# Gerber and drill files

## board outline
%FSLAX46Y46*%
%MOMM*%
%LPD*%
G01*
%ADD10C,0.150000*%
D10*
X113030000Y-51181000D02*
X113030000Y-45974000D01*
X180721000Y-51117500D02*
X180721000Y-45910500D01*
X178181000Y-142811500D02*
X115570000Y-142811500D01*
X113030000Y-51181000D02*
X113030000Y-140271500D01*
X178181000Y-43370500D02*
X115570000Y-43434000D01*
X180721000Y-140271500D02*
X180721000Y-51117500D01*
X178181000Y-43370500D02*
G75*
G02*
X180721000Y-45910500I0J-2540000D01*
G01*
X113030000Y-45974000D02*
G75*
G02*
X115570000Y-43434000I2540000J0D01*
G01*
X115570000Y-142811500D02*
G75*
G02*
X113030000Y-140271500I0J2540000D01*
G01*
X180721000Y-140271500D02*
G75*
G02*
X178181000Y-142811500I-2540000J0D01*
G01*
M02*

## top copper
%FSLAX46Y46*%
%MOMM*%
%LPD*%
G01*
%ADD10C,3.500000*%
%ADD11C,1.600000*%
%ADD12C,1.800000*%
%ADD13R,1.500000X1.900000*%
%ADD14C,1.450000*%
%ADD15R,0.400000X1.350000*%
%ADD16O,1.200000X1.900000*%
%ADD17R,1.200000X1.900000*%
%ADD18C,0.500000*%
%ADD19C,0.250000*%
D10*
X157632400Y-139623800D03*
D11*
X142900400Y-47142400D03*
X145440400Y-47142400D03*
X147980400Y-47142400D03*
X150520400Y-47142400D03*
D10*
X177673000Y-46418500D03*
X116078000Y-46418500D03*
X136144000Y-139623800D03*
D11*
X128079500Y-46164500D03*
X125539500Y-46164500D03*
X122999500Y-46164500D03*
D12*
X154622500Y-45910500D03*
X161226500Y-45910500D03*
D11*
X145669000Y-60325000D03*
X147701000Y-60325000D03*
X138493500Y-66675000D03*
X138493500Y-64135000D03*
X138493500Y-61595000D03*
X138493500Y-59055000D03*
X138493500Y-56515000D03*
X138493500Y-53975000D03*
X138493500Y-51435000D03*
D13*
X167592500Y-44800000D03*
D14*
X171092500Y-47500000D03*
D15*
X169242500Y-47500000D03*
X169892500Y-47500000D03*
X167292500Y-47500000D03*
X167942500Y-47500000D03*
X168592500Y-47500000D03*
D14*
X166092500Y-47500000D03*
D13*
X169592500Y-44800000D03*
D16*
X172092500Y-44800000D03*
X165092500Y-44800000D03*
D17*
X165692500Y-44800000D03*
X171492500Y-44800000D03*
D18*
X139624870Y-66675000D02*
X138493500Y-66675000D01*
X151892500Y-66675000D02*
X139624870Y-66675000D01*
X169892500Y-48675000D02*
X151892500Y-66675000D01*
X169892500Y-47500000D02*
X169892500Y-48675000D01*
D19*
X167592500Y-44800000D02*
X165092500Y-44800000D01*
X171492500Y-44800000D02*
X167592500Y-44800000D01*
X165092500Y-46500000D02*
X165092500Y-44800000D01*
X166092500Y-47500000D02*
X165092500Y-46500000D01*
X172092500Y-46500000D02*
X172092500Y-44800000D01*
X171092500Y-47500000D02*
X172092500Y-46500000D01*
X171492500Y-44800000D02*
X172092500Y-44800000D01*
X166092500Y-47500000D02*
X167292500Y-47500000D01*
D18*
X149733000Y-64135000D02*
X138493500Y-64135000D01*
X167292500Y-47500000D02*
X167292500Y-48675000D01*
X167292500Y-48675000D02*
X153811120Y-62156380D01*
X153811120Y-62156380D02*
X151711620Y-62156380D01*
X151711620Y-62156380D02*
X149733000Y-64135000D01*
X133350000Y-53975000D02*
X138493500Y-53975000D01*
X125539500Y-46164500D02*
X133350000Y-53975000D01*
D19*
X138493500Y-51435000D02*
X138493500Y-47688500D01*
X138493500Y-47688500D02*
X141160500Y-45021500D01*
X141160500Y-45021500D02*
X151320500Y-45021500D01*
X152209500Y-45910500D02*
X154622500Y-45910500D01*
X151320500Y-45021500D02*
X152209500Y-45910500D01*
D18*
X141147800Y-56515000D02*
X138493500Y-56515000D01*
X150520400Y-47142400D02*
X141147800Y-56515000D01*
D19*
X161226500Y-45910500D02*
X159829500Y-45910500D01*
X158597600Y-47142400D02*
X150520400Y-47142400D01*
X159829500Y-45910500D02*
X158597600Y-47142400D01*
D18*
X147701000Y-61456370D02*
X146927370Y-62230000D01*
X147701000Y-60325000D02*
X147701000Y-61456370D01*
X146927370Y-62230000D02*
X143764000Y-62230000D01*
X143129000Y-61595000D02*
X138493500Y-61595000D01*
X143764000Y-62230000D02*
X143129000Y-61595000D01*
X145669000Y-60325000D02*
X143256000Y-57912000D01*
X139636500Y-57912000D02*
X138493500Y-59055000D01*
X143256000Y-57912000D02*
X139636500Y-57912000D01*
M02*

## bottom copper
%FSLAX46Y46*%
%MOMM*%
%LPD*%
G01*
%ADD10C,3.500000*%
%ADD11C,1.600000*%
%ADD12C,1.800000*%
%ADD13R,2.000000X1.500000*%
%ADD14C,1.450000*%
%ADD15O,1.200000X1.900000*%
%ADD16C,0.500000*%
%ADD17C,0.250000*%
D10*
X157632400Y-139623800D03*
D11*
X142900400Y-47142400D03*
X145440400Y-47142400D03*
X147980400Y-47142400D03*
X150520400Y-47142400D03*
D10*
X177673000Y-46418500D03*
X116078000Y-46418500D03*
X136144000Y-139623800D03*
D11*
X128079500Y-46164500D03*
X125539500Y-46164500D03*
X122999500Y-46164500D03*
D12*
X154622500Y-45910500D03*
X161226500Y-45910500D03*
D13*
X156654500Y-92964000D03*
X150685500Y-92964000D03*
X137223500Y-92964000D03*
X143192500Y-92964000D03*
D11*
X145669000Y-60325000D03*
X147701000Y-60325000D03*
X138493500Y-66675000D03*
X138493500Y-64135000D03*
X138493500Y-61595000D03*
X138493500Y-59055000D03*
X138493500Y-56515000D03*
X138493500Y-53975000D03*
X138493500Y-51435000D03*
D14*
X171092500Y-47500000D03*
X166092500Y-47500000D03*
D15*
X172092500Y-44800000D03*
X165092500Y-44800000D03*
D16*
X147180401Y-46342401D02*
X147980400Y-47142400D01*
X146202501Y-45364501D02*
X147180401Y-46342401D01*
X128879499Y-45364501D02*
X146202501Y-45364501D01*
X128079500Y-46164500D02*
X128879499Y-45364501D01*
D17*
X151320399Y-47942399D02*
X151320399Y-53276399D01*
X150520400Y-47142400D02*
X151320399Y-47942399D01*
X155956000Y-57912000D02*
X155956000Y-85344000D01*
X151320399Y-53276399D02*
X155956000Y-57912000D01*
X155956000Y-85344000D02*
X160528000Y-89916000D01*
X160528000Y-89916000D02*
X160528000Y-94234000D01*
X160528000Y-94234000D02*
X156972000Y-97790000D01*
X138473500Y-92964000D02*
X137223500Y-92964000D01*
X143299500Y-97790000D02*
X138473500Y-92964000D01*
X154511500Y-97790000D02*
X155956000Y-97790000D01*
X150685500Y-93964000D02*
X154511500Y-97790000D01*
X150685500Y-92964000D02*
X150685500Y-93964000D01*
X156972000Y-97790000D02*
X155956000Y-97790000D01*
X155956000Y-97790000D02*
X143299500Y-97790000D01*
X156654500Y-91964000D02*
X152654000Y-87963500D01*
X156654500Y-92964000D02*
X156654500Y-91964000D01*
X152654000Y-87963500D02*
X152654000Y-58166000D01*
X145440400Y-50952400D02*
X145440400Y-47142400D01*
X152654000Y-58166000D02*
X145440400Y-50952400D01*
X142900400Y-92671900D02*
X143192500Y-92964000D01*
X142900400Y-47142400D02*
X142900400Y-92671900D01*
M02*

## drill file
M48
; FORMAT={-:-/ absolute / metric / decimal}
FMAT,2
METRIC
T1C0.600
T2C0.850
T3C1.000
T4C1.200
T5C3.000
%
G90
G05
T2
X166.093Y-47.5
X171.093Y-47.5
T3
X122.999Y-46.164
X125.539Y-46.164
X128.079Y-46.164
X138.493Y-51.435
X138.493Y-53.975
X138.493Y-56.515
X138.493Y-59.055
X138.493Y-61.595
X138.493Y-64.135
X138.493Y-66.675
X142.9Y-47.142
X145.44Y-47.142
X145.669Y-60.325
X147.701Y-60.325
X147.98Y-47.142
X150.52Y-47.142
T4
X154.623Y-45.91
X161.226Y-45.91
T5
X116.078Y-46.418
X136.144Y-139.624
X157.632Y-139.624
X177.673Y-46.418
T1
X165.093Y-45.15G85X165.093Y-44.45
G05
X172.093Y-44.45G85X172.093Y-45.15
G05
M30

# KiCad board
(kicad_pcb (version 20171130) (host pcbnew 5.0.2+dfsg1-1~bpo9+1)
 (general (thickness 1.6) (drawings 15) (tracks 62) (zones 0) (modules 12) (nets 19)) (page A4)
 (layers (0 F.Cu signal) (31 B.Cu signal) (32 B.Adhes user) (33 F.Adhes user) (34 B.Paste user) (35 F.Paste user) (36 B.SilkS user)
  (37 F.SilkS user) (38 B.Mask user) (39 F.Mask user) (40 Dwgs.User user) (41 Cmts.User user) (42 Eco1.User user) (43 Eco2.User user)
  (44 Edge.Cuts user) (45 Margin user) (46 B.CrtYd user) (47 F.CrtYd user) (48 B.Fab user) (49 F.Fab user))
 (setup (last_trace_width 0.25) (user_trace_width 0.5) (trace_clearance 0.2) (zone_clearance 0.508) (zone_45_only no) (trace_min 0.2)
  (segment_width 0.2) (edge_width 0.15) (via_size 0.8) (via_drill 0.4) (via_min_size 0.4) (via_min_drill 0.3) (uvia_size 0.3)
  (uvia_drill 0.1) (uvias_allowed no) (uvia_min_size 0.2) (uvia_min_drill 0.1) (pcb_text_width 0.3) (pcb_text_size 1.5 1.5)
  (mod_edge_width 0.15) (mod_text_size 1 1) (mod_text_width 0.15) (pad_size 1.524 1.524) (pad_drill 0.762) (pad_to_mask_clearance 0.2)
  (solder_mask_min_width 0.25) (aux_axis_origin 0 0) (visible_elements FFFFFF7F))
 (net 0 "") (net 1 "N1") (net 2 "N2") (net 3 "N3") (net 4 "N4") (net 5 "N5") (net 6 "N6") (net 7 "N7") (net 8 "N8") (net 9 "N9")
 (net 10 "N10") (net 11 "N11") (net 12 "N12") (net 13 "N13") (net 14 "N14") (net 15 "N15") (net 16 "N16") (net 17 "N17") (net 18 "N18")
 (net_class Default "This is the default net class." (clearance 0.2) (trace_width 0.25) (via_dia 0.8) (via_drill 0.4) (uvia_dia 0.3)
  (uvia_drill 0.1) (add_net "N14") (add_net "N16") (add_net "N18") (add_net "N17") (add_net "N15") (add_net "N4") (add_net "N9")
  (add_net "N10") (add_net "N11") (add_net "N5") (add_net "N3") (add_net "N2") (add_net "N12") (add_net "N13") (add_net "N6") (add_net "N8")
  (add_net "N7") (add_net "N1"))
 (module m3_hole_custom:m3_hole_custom (layer F.Cu) (at 157.6324 139.6238)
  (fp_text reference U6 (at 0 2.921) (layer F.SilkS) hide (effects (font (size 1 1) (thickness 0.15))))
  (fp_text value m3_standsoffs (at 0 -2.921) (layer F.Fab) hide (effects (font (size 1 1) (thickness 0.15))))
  (pad 1 thru_hole circle (at 0 0) (size 3.5 3.5) (drill 3) (layers *.Cu *.Mask) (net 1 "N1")))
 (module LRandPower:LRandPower (layer F.Cu) (at 146.7104 47.1424)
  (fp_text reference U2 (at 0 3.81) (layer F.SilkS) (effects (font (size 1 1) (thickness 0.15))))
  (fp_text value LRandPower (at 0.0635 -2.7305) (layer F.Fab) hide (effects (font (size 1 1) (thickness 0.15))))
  (pad 1 thru_hole circle (at -3.81 0) (size 1.6 1.6) (drill 1) (layers *.Cu *.Mask) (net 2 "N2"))
  (pad 2 thru_hole circle (at -1.27 0) (size 1.6 1.6) (drill 1) (layers *.Cu *.Mask) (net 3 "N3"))
  (pad 3 thru_hole circle (at 1.27 0) (size 1.6 1.6) (drill 1) (layers *.Cu *.Mask) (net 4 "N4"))
  (pad 4 thru_hole circle (at 3.81 0) (size 1.6 1.6) (drill 1) (layers *.Cu *.Mask) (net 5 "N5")))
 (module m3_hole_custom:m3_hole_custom (layer F.Cu) (at 177.673 46.4185)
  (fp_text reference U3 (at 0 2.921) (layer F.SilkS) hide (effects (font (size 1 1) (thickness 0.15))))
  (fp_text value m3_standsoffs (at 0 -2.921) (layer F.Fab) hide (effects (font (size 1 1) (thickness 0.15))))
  (pad 1 thru_hole circle (at 0 0) (size 3.5 3.5) (drill 3) (layers *.Cu *.Mask) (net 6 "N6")))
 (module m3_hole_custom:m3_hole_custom (layer F.Cu) (at 116.078 46.4185)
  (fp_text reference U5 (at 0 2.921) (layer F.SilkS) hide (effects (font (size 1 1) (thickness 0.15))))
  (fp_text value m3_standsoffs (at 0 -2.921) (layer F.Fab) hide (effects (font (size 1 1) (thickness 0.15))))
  (pad 1 thru_hole circle (at 0 0) (size 3.5 3.5) (drill 3) (layers *.Cu *.Mask) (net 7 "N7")))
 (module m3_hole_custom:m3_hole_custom (layer F.Cu) (at 136.144 139.6238)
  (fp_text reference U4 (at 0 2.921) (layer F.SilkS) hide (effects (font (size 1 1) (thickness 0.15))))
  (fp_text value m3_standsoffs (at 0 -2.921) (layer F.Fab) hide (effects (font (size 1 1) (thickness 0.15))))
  (pad 1 thru_hole circle (at 0 0) (size 3.5 3.5) (drill 3) (layers *.Cu *.Mask) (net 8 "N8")))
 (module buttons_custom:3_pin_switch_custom (layer F.Cu) (at 125.5395 46.1645 180)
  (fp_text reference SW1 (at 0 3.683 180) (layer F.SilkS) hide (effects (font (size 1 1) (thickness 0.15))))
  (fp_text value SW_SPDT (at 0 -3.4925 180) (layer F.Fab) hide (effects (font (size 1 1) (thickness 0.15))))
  (pad 1 thru_hole circle (at -2.54 0 180) (size 1.6 1.6) (drill 1) (layers *.Cu *.Mask) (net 4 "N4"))
  (pad 2 thru_hole circle (at 0 0 180) (size 1.6 1.6) (drill 1) (layers *.Cu *.Mask) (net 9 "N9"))
  (pad 3 thru_hole circle (at 2.54 0 180) (size 1.6 1.6) (drill 1) (layers *.Cu *.Mask) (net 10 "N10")))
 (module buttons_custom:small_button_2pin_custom (layer F.Cu) (at 157.9245 45.9105 180)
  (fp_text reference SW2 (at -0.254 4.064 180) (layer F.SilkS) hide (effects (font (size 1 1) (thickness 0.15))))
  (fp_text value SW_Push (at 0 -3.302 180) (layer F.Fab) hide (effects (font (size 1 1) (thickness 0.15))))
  (pad 1 thru_hole circle (at 3.302 0 180) (size 1.8 1.8) (drill 1.2) (layers *.Cu *.Mask) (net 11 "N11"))
  (pad 2 thru_hole circle (at -3.302 0 180) (size 1.8 1.8) (drill 1.2) (layers *.Cu *.Mask) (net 5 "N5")))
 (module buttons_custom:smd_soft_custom (layer B.Cu) (at 153.67 92.964)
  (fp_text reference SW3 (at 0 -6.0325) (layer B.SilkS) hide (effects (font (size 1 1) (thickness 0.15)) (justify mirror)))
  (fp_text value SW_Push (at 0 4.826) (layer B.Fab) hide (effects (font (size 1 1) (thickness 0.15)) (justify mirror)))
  (pad 1 smd rect (at 2.9845 0 270) (size 1.5 2) (layers B.Cu B.Paste B.Mask) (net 3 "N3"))
  (pad 2 smd rect (at -2.9845 0 270) (size 1.5 2) (layers B.Cu B.Paste B.Mask) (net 5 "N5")))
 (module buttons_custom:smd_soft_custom (layer B.Cu) (at 140.208 92.964)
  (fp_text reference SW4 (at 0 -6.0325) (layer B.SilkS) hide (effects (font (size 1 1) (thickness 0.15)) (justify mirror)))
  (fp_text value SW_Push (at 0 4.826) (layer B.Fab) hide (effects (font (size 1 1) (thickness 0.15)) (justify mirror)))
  (pad 2 smd rect (at -2.9845 0 270) (size 1.5 2) (layers B.Cu B.Paste B.Mask) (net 5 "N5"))
  (pad 1 smd rect (at 2.9845 0 270) (size 1.5 2) (layers B.Cu B.Paste B.Mask) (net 2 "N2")))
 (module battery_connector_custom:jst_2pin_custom (layer F.Cu) (at 146.685 60.325)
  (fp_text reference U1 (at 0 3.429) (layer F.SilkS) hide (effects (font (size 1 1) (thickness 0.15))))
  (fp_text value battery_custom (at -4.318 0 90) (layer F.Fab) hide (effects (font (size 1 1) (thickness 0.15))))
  (pad 1 thru_hole circle (at -1.016 0) (size 1.6 1.6) (drill 1) (layers *.Cu *.Mask) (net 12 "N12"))
  (pad 2 thru_hole circle (at 1.016 0) (size 1.6 1.6) (drill 1) (layers *.Cu *.Mask) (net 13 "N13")))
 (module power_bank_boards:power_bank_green (layer F.Cu) (at 138.4935 59.055 90)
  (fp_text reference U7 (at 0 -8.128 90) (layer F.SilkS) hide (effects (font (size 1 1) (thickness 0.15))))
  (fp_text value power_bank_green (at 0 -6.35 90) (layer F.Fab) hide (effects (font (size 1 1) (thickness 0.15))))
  (pad 1 thru_hole circle (at -7.62 0 90) (size 1.6 1.6) (drill 1) (layers *.Cu *.Mask) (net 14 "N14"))
  (pad 2 thru_hole circle (at -5.08 0 90) (size 1.6 1.6) (drill 1) (layers *.Cu *.Mask) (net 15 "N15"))
  (pad 3 thru_hole circle (at -2.54 0 90) (size 1.6 1.6) (drill 1) (layers *.Cu *.Mask) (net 13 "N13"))
  (pad 4 thru_hole circle (at 0 0 90) (size 1.6 1.6) (drill 1) (layers *.Cu *.Mask) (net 12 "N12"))
  (pad 5 thru_hole circle (at 2.54 0 90) (size 1.6 1.6) (drill 1) (layers *.Cu *.Mask) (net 5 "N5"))
  (pad 6 thru_hole circle (at 5.08 0 90) (size 1.6 1.6) (drill 1) (layers *.Cu *.Mask) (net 9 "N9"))
  (pad 7 thru_hole circle (at 7.62 0 90) (size 1.6 1.6) (drill 1) (layers *.Cu *.Mask) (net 11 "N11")))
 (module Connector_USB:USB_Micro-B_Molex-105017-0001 (layer F.Cu) (at 168.5925 46.0375 180)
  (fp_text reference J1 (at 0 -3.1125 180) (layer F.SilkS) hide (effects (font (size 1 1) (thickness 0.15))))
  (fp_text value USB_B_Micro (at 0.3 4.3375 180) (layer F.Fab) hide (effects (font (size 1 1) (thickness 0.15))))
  (pad 6 smd rect (at 1 1.2375 180) (size 1.5 1.9) (layers F.Cu F.Paste F.Mask) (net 15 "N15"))
  (pad 6 thru_hole circle (at -2.5 -1.4625 180) (size 1.45 1.45) (drill 0.85) (layers *.Cu *.Mask) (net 15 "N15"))
  (pad 2 smd rect (at -0.65 -1.4625 180) (size 0.4 1.35) (layers F.Cu F.Paste F.Mask) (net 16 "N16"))
  (pad 1 smd rect (at -1.3 -1.4625 180) (size 0.4 1.35) (layers F.Cu F.Paste F.Mask) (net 14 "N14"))
  (pad 5 smd rect (at 1.3 -1.4625 180) (size 0.4 1.35) (layers F.Cu F.Paste F.Mask) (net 15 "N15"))
  (pad 4 smd rect (at 0.65 -1.4625 180) (size 0.4 1.35) (layers F.Cu F.Paste F.Mask) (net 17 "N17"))
  (pad 3 smd rect (at 0 -1.4625 180) (size 0.4 1.35) (layers F.Cu F.Paste F.Mask) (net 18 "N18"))
  (pad 6 thru_hole circle (at 2.5 -1.4625 180) (size 1.45 1.45) (drill 0.85) (layers *.Cu *.Mask) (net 15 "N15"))
  (pad 6 smd rect (at -1 1.2375 180) (size 1.5 1.9) (layers F.Cu F.Paste F.Mask) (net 15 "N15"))
  (pad 6 thru_hole oval (at -3.5 1.2375) (size 1.2 1.9) (drill oval 0.6 1.3) (layers *.Cu *.Mask) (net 15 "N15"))
  (pad 6 thru_hole oval (at 3.5 1.2375 180) (size 1.2 1.9) (drill oval 0.6 1.3) (layers *.Cu *.Mask) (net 15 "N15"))
  (pad 6 smd rect (at 2.9 1.2375 180) (size 1.2 1.9) (layers F.Cu F.Mask) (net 15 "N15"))
  (pad 6 smd rect (at -2.9 1.2375 180) (size 1.2 1.9) (layers F.Cu F.Mask) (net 15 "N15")))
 (gr_line (start 113.03 51.181) (end 113.03 45.974) (layer Edge.Cuts) (width 0.15))
 (gr_line (start 180.721 51.1175) (end 180.721 45.9105) (layer Edge.Cuts) (width 0.15))
 (gr_line (start 178.181 142.8115) (end 115.57 142.8115) (layer Edge.Cuts) (width 0.15))
 (gr_line (start 113.03 51.181) (end 113.03 140.2715) (layer Edge.Cuts) (width 0.15))
 (gr_line (start 178.181 43.3705) (end 115.57 43.434) (layer Edge.Cuts) (width 0.15))
 (gr_line (start 180.721 140.2715) (end 180.721 51.1175) (layer Edge.Cuts) (width 0.15))
 (gr_arc (start 178.181 45.9105) (end 180.721 45.9105) (angle -90) (layer Edge.Cuts) (width 0.15))
 (gr_arc (start 115.57 45.974) (end 115.57 43.434) (angle -90) (layer Edge.Cuts) (width 0.15))
 (gr_arc (start 115.57 140.2715) (end 113.03 140.2715) (angle -90) (layer Edge.Cuts) (width 0.15))
 (gr_arc (start 178.181 140.2715) (end 178.181 142.8115) (angle -90) (layer Edge.Cuts) (width 0.15))
 (segment (start 139.62487 66.675) (end 138.4935 66.675) (width 0.5) (layer F.Cu) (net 14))
 (segment (start 151.8925 66.675) (end 139.62487 66.675) (width 0.5) (layer F.Cu) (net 14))
 (segment (start 169.8925 48.675) (end 151.8925 66.675) (width 0.5) (layer F.Cu) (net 14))
 (segment (start 169.8925 47.5) (end 169.8925 48.675) (width 0.5) (layer F.Cu) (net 14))
 (segment (start 167.5925 44.8) (end 165.0925 44.8) (width 0.25) (layer F.Cu) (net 15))
 (segment (start 171.4925 44.8) (end 167.5925 44.8) (width 0.25) (layer F.Cu) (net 15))
 (segment (start 165.0925 46.5) (end 165.0925 44.8) (width 0.25) (layer F.Cu) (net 15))
 (segment (start 166.0925 47.5) (end 165.0925 46.5) (width 0.25) (layer F.Cu) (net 15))
 (segment (start 172.0925 46.5) (end 172.0925 44.8) (width 0.25) (layer F.Cu) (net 15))
 (segment (start 171.0925 47.5) (end 172.0925 46.5) (width 0.25) (layer F.Cu) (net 15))
 (segment (start 171.4925 44.8) (end 172.0925 44.8) (width 0.25) (layer F.Cu) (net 15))
 (segment (start 166.0925 47.5) (end 167.2925 47.5) (width 0.25) (layer F.Cu) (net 15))
 (segment (start 149.733 64.135) (end 138.4935 64.135) (width 0.5) (layer F.Cu) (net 15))
 (segment (start 167.2925 47.5) (end 167.2925 48.675) (width 0.5) (layer F.Cu) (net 15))
 (segment (start 167.2925 48.675) (end 153.81112 62.15638) (width 0.5) (layer F.Cu) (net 15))
 (segment (start 153.81112 62.15638) (end 151.71162 62.15638) (width 0.5) (layer F.Cu) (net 15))
 (segment (start 151.71162 62.15638) (end 149.733 64.135) (width 0.5) (layer F.Cu) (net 15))
 (segment (start 147.180401 46.342401) (end 147.9804 47.1424) (width 0.5) (layer B.Cu) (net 4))
 (segment (start 146.202501 45.364501) (end 147.180401 46.342401) (width 0.5) (layer B.Cu) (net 4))
 (segment (start 128.879499 45.364501) (end 146.202501 45.364501) (width 0.5) (layer B.Cu) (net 4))
 (segment (start 128.0795 46.1645) (end 128.879499 45.364501) (width 0.5) (layer B.Cu) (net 4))
 (segment (start 133.35 53.975) (end 138.4935 53.975) (width 0.5) (layer F.Cu) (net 9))
 (segment (start 125.5395 46.1645) (end 133.35 53.975) (width 0.5) (layer F.Cu) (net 9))
 (segment (start 138.4935 51.435) (end 138.4935 47.6885) (width 0.25) (layer F.Cu) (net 11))
 (segment (start 138.4935 47.6885) (end 141.1605 45.0215) (width 0.25) (layer F.Cu) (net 11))
 (segment (start 141.1605 45.0215) (end 151.3205 45.0215) (width 0.25) (layer F.Cu) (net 11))
 (segment (start 152.2095 45.9105) (end 154.6225 45.9105) (width 0.25) (layer F.Cu) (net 11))
 (segment (start 151.3205 45.0215) (end 152.2095 45.9105) (width 0.25) (layer F.Cu) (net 11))
 (segment (start 141.1478 56.515) (end 138.4935 56.515) (width 0.5) (layer F.Cu) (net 5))
 (segment (start 150.5204 47.1424) (end 141.1478 56.515) (width 0.5) (layer F.Cu) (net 5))
 (segment (start 161.2265 45.9105) (end 159.8295 45.9105) (width 0.25) (layer F.Cu) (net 5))
 (segment (start 158.5976 47.1424) (end 150.5204 47.1424) (width 0.25) (layer F.Cu) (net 5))
 (segment (start 159.8295 45.9105) (end 158.5976 47.1424) (width 0.25) (layer F.Cu) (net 5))
 (segment (start 151.320399 47.942399) (end 151.320399 53.276399) (width 0.25) (layer B.Cu) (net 5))
 (segment (start 150.5204 47.1424) (end 151.320399 47.942399) (width 0.25) (layer B.Cu) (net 5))
 (segment (start 155.956 57.912) (end 155.956 85.344) (width 0.25) (layer B.Cu) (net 5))
 (segment (start 151.320399 53.276399) (end 155.956 57.912) (width 0.25) (layer B.Cu) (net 5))
 (segment (start 155.956 85.344) (end 160.528 89.916) (width 0.25) (layer B.Cu) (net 5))
 (segment (start 160.528 89.916) (end 160.528 94.234) (width 0.25) (layer B.Cu) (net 5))
 (segment (start 160.528 94.234) (end 156.972 97.79) (width 0.25) (layer B.Cu) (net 5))
 (segment (start 138.4735 92.964) (end 137.2235 92.964) (width 0.25) (layer B.Cu) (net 5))
 (segment (start 143.2995 97.79) (end 138.4735 92.964) (width 0.25) (layer B.Cu) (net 5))
 (segment (start 154.5115 97.79) (end 155.956 97.79) (width 0.25) (layer B.Cu) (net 5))
 (segment (start 150.6855 93.964) (end 154.5115 97.79) (width 0.25) (layer B.Cu) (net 5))
 (segment (start 150.6855 92.964) (end 150.6855 93.964) (width 0.25) (layer B.Cu) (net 5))
 (segment (start 156.972 97.79) (end 155.956 97.79) (width 0.25) (layer B.Cu) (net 5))
 (segment (start 155.956 97.79) (end 143.2995 97.79) (width 0.25) (layer B.Cu) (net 5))
 (segment (start 156.6545 91.964) (end 152.654 87.9635) (width 0.25) (layer B.Cu) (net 3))
 (segment (start 156.6545 92.964) (end 156.6545 91.964) (width 0.25) (layer B.Cu) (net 3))
 (segment (start 152.654 87.9635) (end 152.654 58.166) (width 0.25) (layer B.Cu) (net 3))
 (segment (start 145.4404 50.9524) (end 145.4404 47.1424) (width 0.25) (layer B.Cu) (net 3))
 (segment (start 152.654 58.166) (end 145.4404 50.9524) (width 0.25) (layer B.Cu) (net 3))
 (segment (start 142.9004 92.6719) (end 143.1925 92.964) (width 0.25) (layer B.Cu) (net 2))
 (segment (start 142.9004 47.1424) (end 142.9004 92.6719) (width 0.25) (layer B.Cu) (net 2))
 (segment (start 147.701 61.45637) (end 146.92737 62.23) (width 0.5) (layer F.Cu) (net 13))
 (segment (start 147.701 60.325) (end 147.701 61.45637) (width 0.5) (layer F.Cu) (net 13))
 (segment (start 146.92737 62.23) (end 143.764 62.23) (width 0.5) (layer F.Cu) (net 13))
 (segment (start 143.129 61.595) (end 138.4935 61.595) (width 0.5) (layer F.Cu) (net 13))
 (segment (start 143.764 62.23) (end 143.129 61.595) (width 0.5) (layer F.Cu) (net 13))
 (segment (start 145.669 60.325) (end 143.256 57.912) (width 0.5) (layer F.Cu) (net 12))
 (segment (start 139.6365 57.912) (end 138.4935 59.055) (width 0.5) (layer F.Cu) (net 12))
 (segment (start 143.256 57.912) (end 139.6365 57.912) (width 0.5) (layer F.Cu) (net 12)))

